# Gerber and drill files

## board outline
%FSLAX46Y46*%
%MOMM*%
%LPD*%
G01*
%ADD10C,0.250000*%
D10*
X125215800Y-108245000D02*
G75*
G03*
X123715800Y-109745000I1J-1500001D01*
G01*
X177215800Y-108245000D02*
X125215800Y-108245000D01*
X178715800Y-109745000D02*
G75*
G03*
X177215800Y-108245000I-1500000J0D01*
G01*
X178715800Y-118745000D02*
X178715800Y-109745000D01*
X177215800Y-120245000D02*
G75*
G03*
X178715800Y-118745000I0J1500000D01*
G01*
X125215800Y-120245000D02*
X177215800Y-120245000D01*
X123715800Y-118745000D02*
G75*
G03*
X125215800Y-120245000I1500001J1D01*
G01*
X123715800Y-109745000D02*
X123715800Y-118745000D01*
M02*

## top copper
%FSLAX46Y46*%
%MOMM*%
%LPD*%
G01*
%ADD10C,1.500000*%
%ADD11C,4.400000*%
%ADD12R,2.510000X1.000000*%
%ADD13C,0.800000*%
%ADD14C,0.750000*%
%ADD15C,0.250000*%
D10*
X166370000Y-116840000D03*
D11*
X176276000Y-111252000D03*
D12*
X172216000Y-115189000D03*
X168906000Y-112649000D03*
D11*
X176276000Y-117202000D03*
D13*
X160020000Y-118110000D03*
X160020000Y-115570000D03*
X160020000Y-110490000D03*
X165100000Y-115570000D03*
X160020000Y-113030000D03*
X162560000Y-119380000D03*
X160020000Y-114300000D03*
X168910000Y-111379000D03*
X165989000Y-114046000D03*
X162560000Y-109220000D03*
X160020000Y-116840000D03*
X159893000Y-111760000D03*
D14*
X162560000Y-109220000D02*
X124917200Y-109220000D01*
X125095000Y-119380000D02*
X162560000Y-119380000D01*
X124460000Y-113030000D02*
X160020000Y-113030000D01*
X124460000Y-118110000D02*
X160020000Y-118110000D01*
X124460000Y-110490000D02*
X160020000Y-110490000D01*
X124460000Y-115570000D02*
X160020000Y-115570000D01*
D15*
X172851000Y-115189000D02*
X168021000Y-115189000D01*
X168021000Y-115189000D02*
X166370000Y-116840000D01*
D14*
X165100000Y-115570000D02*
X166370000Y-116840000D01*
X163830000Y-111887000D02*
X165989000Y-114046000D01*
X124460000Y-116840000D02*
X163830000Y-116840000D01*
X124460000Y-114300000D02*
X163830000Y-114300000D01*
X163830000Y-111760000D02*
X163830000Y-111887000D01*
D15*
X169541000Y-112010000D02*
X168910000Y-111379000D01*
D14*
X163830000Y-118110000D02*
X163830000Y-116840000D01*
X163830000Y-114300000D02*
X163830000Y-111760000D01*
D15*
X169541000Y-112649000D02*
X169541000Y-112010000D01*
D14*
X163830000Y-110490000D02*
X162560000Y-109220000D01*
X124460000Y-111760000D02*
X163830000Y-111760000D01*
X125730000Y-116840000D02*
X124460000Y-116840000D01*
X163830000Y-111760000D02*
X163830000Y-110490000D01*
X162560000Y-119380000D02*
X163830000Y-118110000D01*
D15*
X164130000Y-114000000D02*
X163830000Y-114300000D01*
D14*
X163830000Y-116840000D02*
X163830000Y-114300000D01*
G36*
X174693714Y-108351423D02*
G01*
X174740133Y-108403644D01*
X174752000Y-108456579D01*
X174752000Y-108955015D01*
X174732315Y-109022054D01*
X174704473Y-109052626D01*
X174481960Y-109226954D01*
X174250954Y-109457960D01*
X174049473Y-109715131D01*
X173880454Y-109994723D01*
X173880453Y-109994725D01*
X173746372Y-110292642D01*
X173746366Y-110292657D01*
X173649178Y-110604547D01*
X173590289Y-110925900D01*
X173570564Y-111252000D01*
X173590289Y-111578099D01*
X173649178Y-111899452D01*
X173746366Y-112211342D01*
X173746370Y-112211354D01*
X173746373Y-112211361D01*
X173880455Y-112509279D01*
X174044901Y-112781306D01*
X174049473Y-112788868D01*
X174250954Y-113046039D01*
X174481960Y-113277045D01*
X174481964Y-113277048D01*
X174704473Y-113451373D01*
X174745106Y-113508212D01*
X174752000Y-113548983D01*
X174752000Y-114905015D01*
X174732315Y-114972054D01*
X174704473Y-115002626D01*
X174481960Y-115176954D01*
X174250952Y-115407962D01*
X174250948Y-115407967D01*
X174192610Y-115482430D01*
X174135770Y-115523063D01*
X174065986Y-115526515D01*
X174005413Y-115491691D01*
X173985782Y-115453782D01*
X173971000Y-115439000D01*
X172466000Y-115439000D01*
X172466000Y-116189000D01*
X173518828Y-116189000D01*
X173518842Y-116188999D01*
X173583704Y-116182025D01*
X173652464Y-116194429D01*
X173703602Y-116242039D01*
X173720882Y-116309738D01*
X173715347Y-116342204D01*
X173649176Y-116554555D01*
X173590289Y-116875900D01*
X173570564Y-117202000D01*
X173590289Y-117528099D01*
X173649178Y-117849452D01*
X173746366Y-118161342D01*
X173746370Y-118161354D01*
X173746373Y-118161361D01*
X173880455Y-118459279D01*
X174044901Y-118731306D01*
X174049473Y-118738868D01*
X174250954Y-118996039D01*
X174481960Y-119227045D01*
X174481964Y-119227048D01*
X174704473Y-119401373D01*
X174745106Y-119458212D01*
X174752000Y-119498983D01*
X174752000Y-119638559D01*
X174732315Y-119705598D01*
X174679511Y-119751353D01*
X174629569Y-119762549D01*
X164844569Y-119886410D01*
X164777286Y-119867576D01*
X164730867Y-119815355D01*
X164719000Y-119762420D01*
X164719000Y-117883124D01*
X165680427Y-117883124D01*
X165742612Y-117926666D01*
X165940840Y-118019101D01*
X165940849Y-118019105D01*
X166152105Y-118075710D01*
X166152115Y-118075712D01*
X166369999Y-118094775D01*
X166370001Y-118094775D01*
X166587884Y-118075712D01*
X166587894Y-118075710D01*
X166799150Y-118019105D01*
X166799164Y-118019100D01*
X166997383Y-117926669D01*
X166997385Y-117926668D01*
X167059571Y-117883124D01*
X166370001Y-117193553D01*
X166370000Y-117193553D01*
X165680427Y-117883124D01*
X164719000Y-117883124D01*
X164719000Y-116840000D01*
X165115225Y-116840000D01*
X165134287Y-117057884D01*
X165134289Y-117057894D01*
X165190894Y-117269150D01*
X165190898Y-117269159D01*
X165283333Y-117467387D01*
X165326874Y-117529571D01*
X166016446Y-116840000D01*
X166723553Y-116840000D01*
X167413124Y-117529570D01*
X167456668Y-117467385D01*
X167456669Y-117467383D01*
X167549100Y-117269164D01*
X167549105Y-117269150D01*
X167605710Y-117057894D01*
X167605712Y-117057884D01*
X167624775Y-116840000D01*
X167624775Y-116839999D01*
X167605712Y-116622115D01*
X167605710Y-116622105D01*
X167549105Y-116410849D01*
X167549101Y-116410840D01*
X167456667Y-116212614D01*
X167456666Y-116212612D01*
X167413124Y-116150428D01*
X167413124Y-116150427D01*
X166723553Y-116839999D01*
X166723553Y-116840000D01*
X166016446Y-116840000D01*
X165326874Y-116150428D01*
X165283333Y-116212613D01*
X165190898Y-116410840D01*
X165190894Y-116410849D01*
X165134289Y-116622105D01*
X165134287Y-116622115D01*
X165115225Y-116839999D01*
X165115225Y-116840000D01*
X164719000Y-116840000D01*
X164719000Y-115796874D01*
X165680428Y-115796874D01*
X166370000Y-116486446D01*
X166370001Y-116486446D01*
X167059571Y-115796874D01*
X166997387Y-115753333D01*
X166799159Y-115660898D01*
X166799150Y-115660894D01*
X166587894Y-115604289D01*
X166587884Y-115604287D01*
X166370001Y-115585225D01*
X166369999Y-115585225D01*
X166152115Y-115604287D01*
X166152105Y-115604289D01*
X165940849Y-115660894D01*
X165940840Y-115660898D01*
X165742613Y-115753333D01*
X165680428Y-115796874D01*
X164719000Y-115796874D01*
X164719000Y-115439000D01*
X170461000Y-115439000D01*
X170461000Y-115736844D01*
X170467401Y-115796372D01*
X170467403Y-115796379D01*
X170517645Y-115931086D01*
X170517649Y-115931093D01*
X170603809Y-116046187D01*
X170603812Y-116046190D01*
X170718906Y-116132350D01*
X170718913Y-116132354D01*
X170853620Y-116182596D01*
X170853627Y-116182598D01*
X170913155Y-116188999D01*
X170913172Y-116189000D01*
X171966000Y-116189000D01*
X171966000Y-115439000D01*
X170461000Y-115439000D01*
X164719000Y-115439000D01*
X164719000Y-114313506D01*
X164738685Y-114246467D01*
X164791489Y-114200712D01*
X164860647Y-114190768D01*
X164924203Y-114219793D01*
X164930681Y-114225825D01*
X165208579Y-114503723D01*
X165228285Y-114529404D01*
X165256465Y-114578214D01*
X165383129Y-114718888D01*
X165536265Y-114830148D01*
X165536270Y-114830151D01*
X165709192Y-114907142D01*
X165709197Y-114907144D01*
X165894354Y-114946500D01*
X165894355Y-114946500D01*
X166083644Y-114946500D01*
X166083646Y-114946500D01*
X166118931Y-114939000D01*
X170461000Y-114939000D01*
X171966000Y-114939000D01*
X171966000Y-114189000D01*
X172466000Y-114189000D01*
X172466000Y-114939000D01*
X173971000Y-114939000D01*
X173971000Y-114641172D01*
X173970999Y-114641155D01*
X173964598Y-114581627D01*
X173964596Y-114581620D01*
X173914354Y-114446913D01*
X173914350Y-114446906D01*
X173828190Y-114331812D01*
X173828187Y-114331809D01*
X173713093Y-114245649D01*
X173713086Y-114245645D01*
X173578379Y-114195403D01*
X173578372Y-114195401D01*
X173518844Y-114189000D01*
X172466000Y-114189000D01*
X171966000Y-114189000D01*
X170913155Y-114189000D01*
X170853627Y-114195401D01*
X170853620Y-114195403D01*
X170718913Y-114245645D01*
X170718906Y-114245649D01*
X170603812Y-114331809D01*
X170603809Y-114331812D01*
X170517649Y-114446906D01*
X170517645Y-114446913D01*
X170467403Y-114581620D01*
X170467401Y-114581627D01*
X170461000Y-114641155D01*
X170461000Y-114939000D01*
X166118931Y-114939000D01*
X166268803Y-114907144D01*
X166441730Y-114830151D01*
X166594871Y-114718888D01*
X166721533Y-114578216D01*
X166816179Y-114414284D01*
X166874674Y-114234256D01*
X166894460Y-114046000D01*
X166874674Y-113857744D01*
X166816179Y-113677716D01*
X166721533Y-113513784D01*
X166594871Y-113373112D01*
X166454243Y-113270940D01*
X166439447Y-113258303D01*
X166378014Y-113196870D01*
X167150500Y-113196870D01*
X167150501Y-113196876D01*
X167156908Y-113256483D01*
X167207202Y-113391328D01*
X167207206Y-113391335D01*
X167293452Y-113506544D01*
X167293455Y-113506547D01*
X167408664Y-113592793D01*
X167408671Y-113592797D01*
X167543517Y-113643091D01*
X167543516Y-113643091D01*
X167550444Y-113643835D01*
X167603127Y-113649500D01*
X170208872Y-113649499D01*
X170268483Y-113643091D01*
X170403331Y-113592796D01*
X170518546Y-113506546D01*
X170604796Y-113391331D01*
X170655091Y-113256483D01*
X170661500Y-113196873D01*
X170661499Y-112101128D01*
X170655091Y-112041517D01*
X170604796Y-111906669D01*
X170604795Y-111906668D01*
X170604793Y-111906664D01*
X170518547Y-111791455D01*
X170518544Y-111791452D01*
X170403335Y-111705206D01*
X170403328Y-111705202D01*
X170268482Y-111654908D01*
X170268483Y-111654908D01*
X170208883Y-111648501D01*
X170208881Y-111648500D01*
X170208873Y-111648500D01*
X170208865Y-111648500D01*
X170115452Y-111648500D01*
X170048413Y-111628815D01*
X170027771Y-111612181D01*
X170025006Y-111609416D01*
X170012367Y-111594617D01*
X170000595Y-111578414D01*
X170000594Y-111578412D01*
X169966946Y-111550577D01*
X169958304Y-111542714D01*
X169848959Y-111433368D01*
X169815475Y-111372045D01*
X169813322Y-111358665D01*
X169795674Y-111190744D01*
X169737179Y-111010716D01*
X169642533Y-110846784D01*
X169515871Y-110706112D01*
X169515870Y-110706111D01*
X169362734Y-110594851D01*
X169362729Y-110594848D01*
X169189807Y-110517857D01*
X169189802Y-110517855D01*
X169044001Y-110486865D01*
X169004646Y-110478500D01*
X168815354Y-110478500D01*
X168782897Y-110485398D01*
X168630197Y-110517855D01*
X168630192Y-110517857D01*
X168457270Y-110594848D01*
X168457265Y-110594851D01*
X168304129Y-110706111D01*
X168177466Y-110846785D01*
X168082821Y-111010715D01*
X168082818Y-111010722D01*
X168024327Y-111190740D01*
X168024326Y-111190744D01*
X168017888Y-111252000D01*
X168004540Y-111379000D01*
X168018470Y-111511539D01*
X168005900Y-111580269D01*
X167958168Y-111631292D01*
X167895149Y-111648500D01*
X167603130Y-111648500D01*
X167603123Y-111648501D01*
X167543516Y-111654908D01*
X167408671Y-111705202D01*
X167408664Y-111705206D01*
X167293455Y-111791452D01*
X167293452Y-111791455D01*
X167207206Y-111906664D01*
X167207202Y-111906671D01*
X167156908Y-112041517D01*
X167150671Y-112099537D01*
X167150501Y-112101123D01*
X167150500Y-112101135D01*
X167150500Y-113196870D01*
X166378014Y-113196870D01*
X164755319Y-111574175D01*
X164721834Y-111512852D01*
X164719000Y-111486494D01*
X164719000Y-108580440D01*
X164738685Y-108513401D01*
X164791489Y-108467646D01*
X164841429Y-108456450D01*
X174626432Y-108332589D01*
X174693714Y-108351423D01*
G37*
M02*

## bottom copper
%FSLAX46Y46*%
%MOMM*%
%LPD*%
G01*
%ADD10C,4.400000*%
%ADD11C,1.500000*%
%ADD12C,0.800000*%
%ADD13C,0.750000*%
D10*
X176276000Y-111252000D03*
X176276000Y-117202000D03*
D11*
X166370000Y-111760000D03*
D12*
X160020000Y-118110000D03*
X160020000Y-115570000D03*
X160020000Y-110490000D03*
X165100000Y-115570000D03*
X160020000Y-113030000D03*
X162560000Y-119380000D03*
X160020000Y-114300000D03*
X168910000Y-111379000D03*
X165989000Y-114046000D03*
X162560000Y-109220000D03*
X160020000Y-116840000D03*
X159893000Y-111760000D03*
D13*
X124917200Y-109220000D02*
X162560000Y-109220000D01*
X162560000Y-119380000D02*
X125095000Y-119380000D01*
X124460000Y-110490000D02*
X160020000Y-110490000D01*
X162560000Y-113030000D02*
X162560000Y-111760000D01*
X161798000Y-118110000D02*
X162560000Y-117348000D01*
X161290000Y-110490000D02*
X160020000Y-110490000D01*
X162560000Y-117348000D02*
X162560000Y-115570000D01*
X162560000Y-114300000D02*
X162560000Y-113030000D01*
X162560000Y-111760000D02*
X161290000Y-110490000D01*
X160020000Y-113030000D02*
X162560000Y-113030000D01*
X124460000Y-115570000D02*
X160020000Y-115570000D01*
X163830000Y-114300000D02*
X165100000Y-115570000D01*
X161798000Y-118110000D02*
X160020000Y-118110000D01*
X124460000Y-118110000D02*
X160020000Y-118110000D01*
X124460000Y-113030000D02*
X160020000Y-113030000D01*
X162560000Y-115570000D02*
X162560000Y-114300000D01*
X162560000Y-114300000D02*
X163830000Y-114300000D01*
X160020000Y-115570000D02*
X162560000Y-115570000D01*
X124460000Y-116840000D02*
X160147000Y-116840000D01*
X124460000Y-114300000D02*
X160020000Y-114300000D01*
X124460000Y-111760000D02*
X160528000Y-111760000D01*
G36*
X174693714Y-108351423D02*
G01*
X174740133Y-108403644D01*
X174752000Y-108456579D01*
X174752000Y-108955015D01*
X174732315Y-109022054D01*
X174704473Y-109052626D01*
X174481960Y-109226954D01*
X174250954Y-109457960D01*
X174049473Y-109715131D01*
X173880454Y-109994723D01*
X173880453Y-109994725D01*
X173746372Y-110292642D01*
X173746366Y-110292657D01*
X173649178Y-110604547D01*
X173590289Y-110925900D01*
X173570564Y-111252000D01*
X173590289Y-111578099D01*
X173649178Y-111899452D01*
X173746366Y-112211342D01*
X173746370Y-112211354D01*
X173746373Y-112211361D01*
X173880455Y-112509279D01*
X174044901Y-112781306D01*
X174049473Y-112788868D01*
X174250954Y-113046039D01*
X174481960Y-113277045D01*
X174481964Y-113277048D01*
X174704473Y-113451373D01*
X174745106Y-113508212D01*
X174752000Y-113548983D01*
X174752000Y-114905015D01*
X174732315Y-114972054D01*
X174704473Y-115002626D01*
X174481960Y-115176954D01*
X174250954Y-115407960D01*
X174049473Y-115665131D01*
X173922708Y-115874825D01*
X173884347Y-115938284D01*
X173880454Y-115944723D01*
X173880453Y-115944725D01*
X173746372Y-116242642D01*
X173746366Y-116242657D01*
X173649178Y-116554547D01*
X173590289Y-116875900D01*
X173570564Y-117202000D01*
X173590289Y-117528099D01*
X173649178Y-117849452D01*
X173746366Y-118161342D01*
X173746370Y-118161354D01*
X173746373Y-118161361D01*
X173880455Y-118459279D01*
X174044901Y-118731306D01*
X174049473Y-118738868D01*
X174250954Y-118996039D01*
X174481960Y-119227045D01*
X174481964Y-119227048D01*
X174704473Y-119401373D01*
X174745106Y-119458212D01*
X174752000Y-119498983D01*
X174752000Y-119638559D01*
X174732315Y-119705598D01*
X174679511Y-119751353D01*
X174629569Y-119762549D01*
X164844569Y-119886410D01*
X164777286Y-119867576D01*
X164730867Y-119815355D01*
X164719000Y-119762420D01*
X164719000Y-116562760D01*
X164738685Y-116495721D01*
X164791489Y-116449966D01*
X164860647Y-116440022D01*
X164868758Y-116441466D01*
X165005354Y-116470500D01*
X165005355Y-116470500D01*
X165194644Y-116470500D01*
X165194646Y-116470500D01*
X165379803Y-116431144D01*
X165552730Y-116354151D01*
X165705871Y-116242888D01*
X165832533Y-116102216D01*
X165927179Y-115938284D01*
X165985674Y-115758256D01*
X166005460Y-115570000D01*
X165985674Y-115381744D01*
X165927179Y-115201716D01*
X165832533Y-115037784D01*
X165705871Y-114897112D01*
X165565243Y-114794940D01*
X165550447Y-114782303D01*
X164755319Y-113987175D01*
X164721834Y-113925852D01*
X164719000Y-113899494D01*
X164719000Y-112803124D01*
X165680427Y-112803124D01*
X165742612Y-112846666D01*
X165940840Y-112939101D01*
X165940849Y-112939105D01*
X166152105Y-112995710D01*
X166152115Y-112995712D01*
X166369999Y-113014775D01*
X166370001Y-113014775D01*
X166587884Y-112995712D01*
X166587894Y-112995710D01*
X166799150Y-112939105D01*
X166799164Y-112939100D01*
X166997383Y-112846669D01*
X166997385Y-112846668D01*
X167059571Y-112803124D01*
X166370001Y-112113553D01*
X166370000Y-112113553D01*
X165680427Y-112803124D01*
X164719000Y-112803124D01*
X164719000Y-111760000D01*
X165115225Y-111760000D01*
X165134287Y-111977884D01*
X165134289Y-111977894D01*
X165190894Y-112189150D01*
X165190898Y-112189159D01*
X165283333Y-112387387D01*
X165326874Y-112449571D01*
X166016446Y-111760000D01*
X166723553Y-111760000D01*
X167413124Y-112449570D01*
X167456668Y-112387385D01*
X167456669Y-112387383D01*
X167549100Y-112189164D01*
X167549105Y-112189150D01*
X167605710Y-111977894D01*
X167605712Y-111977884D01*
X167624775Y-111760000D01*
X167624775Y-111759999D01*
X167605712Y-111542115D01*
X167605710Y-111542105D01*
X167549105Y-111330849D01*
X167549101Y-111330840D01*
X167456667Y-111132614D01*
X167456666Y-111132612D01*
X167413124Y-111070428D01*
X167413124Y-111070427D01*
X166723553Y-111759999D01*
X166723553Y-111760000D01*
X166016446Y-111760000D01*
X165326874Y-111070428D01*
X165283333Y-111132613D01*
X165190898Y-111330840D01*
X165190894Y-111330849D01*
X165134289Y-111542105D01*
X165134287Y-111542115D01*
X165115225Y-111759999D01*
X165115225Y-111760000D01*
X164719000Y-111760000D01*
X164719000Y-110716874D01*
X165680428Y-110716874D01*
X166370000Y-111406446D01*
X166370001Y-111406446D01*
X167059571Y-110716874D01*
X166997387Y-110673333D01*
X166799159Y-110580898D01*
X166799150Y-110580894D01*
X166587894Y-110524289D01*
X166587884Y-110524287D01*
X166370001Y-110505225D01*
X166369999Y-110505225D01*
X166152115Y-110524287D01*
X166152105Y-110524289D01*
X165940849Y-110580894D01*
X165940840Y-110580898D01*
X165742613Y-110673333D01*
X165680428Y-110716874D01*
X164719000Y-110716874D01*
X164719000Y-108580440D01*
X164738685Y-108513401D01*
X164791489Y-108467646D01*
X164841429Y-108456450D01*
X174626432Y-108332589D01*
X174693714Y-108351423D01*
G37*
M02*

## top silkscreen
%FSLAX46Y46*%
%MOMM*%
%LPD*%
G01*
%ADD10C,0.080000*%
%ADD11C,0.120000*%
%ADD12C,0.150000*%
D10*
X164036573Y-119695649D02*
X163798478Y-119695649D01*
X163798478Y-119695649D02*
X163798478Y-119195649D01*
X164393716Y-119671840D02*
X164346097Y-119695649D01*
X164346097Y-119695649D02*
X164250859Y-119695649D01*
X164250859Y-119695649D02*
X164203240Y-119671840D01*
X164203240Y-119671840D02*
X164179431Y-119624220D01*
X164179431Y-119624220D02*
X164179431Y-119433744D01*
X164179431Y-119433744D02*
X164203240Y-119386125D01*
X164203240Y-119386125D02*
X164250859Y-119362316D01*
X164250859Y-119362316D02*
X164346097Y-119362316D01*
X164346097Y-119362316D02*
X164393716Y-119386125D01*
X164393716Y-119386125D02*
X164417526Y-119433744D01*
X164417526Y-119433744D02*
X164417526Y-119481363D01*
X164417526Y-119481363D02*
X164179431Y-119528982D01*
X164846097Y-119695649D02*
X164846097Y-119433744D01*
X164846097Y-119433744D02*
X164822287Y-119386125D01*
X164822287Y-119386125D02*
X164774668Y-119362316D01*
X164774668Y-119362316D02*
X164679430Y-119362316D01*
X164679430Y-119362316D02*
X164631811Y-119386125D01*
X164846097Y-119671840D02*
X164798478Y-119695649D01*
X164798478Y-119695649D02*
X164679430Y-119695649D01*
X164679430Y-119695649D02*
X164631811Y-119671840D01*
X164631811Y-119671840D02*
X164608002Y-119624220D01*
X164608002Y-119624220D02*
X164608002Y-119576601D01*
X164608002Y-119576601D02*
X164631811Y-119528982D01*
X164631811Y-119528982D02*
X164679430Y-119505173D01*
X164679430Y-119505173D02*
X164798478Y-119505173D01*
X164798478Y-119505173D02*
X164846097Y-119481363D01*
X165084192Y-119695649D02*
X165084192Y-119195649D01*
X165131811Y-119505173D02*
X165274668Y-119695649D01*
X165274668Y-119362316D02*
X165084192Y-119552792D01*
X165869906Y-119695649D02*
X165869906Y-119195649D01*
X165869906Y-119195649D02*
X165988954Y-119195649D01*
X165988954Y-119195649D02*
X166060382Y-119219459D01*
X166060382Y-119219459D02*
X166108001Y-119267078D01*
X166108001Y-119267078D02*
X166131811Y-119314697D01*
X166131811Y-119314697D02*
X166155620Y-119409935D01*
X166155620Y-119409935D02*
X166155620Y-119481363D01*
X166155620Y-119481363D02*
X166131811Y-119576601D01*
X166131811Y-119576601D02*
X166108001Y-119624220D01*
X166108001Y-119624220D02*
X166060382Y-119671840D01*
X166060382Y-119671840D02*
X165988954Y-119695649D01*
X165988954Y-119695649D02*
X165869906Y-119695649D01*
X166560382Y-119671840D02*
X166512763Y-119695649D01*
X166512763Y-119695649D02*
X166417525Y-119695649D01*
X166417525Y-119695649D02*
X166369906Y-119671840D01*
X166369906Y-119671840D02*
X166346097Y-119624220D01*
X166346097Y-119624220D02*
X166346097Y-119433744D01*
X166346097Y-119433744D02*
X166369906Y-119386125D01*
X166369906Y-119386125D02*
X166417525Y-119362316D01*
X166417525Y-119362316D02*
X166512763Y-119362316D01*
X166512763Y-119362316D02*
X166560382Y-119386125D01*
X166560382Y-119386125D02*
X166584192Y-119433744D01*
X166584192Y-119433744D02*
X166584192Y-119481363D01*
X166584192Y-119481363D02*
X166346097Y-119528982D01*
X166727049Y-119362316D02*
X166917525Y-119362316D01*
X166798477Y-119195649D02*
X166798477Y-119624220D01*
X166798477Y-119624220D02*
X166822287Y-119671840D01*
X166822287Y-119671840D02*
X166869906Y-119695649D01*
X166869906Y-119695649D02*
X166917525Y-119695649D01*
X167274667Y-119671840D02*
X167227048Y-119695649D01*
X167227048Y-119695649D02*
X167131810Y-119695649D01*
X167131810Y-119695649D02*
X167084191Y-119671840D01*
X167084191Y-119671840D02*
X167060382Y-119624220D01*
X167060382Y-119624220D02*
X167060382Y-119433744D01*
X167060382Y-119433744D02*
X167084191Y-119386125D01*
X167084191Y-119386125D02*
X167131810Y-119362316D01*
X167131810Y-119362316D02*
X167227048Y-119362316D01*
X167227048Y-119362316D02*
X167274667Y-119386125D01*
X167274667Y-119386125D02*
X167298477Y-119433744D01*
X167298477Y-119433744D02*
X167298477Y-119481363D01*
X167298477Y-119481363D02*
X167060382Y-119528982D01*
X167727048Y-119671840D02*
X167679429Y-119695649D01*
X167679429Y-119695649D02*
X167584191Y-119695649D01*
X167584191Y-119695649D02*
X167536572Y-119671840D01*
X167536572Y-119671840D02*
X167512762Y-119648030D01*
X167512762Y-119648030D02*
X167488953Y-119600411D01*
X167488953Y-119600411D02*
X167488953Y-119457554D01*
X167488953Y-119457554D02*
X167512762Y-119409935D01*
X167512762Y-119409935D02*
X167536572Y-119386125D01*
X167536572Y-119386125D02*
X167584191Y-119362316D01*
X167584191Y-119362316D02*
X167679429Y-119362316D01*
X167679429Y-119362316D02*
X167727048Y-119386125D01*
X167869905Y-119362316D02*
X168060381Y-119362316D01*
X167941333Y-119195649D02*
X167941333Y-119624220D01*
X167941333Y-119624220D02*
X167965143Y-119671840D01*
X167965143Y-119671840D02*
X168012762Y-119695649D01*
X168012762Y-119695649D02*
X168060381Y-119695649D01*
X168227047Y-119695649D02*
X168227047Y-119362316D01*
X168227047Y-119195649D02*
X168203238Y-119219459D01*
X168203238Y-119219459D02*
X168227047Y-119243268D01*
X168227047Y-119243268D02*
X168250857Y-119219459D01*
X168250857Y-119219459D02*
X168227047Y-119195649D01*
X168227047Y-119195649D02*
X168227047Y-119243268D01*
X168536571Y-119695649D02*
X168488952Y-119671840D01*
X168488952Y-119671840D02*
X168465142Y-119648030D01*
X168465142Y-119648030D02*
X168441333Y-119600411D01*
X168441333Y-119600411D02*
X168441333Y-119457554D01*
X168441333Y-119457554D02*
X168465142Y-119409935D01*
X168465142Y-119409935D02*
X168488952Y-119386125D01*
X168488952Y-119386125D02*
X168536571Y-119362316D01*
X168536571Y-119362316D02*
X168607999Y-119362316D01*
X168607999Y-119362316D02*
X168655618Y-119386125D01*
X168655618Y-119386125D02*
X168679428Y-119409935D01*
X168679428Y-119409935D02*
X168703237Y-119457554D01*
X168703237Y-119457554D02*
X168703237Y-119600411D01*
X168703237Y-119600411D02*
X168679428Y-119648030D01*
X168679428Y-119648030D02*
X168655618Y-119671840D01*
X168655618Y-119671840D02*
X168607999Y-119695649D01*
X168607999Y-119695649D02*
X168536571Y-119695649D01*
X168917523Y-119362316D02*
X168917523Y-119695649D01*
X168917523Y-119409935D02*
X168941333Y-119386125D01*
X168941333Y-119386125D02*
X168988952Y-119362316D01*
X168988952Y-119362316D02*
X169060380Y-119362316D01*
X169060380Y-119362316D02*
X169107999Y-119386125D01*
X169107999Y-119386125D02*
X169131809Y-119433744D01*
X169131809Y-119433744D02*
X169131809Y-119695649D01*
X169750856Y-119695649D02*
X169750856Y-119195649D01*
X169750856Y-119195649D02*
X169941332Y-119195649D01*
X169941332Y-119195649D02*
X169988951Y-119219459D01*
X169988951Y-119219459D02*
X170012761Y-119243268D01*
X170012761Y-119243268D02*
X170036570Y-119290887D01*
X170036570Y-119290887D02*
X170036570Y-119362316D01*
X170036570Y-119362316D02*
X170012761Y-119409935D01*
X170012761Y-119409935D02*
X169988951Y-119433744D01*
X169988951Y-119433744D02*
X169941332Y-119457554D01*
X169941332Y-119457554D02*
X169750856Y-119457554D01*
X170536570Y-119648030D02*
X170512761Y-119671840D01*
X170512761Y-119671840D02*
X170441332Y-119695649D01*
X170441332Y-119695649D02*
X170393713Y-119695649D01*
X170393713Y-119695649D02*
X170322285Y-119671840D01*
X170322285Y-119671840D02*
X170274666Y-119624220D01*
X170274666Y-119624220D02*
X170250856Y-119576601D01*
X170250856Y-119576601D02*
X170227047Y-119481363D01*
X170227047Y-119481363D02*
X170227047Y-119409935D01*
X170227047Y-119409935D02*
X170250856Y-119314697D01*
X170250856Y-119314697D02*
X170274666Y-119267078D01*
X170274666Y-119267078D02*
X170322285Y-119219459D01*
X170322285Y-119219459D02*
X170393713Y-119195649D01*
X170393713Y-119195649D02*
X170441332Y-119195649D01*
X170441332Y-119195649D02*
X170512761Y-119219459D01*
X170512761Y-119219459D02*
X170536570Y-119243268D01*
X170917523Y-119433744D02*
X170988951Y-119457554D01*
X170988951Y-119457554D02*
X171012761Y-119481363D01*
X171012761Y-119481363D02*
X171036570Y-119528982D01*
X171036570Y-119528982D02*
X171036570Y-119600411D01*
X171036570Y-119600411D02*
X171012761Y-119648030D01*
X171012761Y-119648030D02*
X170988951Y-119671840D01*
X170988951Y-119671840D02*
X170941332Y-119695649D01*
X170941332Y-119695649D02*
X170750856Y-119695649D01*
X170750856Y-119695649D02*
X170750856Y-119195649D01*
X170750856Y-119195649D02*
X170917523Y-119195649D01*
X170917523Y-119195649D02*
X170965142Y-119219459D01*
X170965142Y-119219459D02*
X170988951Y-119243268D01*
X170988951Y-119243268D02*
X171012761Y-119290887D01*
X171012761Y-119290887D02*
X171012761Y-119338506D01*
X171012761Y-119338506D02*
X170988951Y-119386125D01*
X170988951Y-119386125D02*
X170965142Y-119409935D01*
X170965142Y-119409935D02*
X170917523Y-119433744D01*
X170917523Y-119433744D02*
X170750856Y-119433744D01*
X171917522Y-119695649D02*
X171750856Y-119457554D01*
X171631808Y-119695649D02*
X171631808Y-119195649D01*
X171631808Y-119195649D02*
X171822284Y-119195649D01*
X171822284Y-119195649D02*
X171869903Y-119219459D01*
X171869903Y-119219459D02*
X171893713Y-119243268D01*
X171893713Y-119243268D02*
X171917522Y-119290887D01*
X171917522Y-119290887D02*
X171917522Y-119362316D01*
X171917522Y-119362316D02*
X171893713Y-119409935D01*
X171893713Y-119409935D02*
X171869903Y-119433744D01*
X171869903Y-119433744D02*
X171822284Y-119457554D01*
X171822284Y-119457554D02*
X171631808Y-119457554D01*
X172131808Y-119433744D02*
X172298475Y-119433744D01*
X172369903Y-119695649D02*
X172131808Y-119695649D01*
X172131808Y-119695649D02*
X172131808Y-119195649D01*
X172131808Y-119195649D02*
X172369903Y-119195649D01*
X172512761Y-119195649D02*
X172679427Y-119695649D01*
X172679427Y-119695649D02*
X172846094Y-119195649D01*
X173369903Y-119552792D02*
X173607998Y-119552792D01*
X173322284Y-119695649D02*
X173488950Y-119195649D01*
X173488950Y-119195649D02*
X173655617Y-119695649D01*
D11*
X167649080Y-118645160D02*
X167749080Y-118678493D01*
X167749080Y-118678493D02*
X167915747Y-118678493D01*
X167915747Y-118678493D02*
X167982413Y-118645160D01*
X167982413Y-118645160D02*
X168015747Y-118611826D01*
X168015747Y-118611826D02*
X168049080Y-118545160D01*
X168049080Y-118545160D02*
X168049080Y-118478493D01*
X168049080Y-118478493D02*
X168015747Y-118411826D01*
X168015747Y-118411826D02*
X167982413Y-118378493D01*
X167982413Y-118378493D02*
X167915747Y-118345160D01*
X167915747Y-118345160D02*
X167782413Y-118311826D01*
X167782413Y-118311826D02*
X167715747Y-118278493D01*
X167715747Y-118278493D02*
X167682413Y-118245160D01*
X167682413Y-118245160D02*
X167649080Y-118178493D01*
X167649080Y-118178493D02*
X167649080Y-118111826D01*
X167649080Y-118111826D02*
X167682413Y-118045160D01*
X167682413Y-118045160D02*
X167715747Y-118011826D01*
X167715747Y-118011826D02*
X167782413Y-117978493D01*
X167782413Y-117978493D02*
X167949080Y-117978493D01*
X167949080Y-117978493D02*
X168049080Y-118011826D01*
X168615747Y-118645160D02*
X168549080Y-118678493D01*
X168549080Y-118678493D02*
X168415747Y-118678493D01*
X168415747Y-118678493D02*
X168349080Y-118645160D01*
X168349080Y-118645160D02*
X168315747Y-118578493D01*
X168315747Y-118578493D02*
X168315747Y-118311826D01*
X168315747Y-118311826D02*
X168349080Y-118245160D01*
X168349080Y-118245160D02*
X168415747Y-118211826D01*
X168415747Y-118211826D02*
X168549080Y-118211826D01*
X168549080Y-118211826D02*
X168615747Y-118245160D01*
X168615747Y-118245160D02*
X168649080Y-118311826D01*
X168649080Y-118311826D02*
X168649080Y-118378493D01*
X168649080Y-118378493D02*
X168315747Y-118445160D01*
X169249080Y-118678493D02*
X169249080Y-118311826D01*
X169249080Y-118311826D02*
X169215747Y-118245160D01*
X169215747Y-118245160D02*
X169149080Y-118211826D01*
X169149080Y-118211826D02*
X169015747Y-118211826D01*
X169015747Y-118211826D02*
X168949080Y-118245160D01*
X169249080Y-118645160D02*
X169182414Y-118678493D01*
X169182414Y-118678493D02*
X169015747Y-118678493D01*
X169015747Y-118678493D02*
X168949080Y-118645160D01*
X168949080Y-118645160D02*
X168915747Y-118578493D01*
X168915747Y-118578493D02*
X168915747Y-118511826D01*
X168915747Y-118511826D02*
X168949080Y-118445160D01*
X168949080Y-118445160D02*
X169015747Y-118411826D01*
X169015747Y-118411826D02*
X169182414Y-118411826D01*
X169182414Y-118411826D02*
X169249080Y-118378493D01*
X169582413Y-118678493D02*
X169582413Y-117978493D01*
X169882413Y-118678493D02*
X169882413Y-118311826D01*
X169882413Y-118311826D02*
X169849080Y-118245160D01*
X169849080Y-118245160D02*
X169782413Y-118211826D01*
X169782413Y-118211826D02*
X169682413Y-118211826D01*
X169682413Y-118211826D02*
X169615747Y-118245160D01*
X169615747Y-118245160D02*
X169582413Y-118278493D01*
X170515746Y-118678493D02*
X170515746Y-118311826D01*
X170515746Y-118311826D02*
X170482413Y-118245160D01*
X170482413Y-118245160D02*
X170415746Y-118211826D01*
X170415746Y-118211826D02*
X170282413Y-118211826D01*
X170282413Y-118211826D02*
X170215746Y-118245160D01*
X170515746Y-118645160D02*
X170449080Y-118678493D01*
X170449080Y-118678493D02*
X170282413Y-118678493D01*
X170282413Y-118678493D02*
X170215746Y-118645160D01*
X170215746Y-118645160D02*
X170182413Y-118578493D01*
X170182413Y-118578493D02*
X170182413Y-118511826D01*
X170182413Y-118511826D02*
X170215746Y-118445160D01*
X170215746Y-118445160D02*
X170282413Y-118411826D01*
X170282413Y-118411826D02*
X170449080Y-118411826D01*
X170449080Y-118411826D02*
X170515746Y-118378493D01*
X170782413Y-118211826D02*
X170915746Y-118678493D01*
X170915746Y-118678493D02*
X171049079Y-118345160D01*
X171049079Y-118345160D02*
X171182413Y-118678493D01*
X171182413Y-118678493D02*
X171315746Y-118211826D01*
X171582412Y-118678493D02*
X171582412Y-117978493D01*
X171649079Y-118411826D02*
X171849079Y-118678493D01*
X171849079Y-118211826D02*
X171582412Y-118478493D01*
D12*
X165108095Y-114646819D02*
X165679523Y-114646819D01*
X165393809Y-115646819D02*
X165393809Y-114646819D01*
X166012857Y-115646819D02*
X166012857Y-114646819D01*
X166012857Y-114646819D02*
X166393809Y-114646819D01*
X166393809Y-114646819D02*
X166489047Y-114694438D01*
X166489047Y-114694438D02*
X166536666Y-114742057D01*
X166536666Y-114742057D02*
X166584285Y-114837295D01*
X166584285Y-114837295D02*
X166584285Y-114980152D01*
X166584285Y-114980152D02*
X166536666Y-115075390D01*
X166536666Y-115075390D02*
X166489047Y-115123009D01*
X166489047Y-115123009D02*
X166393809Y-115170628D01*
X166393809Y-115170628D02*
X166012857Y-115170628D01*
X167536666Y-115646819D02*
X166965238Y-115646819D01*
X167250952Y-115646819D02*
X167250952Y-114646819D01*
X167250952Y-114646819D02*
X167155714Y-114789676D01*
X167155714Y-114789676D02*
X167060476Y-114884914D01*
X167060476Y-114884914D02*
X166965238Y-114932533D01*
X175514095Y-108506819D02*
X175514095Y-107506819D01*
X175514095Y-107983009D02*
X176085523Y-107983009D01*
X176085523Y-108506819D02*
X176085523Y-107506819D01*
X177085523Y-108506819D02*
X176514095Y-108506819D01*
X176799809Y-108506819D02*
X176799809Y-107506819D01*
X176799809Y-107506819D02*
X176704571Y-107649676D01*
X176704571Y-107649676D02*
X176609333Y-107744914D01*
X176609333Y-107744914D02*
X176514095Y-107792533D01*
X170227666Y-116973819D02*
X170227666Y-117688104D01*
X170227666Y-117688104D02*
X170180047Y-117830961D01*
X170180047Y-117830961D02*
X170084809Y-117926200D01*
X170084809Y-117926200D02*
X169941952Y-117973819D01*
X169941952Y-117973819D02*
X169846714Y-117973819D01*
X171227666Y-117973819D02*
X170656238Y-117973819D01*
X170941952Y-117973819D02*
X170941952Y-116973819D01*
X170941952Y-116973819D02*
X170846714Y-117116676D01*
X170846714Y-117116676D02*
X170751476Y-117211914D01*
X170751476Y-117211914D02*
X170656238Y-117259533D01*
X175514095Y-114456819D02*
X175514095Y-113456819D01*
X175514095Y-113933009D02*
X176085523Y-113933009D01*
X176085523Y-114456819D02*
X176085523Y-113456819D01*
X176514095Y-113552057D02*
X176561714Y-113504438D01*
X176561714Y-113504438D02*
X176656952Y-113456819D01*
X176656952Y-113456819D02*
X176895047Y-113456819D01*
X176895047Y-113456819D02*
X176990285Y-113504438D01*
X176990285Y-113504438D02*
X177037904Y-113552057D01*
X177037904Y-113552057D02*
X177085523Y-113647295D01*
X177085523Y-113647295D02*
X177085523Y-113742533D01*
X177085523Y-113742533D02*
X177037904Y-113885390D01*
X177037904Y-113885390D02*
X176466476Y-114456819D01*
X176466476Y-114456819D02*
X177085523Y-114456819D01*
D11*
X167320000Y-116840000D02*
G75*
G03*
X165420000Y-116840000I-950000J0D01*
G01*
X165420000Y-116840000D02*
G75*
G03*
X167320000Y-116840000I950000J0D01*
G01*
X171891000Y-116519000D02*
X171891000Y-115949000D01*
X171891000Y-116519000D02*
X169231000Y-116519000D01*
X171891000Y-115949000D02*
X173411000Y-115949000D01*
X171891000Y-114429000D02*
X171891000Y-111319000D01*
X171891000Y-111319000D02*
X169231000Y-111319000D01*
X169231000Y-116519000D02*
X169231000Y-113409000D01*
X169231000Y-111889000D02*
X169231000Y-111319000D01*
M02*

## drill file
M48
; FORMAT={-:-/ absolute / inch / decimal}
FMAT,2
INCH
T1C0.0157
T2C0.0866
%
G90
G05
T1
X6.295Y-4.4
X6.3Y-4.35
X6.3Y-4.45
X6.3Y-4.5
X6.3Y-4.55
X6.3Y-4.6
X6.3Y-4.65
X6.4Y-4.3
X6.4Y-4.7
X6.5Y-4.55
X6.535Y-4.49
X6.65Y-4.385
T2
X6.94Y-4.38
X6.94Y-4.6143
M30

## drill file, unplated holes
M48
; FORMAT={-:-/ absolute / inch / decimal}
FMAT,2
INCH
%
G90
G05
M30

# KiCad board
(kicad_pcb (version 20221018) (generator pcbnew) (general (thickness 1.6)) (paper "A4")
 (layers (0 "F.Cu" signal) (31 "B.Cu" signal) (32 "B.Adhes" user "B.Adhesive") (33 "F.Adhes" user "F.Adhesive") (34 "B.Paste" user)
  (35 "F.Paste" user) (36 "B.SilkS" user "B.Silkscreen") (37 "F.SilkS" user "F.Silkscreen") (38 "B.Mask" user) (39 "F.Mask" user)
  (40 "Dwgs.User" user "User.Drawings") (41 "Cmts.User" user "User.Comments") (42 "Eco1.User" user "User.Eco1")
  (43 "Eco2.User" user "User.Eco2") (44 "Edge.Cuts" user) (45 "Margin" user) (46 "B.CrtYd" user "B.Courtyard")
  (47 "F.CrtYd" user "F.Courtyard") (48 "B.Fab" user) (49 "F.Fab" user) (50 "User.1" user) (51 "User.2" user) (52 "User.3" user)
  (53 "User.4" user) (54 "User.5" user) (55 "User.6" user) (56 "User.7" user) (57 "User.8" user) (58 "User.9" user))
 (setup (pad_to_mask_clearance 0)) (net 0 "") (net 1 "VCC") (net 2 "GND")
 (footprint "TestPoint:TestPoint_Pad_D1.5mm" (layer "F.Cu") (at 166.37 116.84)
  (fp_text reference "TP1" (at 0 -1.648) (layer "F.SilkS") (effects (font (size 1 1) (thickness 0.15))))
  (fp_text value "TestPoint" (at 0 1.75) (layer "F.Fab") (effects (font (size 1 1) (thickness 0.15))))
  (fp_circle (center 0 0) (end 0 0.95) (stroke (width 0.12) (type solid)) (fill none) (layer "F.SilkS"))
  (pad "1" smd circle (at 0 0) (size 1.5 1.5) (layers "F.Cu" "F.Mask") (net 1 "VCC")))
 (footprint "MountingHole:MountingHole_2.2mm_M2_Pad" (layer "F.Cu") (at 176.276 111.252)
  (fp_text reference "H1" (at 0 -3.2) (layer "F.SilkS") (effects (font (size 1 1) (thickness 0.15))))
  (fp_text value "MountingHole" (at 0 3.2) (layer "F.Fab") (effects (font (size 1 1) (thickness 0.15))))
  (pad "1" thru_hole circle (at 0 0) (size 4.4 4.4) (drill 2.2) (layers "*.Cu" "*.Mask")))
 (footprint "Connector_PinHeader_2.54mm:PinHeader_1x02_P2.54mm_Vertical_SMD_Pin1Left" (layer "F.Cu") (at 170.561 113.919 180)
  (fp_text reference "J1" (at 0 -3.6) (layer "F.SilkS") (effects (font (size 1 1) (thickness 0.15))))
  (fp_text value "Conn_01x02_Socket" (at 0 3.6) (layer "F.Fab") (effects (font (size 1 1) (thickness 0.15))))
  (fp_line (start -1.33 -2.6) (end -1.33 -2.03) (stroke (width 0.12) (type solid)) (layer "F.SilkS"))
  (fp_line (start -1.33 -2.6) (end 1.33 -2.6) (stroke (width 0.12) (type solid)) (layer "F.SilkS"))
  (fp_line (start -1.33 -2.03) (end -2.85 -2.03) (stroke (width 0.12) (type solid)) (layer "F.SilkS"))
  (fp_line (start -1.33 -0.51) (end -1.33 2.6) (stroke (width 0.12) (type solid)) (layer "F.SilkS"))
  (fp_line (start -1.33 2.6) (end 1.33 2.6) (stroke (width 0.12) (type solid)) (layer "F.SilkS"))
  (fp_line (start 1.33 -2.6) (end 1.33 0.51) (stroke (width 0.12) (type solid)) (layer "F.SilkS"))
  (fp_line (start 1.33 2.03) (end 1.33 2.6) (stroke (width 0.12) (type solid)) (layer "F.SilkS"))
  (pad "1" smd rect (at -1.655 -1.27 180) (size 2.51 1) (layers "F.Cu" "F.Paste" "F.Mask") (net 1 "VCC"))
  (pad "2" smd rect (at 1.655 1.27 180) (size 2.51 1) (layers "F.Cu" "F.Paste" "F.Mask") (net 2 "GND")))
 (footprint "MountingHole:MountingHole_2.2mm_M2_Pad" (layer "F.Cu") (at 176.276 117.202)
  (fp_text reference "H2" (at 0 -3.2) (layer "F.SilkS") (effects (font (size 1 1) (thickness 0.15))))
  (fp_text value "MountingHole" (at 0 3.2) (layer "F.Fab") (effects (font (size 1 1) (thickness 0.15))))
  (pad "1" thru_hole circle (at 0 0) (size 4.4 4.4) (drill 2.2) (layers "*.Cu" "*.Mask")))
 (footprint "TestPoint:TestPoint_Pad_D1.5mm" (layer "B.Cu") (at 166.37 111.76 180)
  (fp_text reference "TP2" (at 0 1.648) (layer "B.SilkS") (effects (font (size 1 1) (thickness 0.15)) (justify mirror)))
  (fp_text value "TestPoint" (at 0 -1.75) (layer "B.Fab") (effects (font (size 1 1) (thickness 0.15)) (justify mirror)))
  (pad "1" smd circle (at 0 0 180) (size 1.5 1.5) (layers "B.Cu" "B.Mask") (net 2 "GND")))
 (gr_arc (start 123.7158 109.745) (mid 124.15514 108.68434) (end 125.2158 108.245) (stroke (width 0.25) (type solid)) (layer "Edge.Cuts"))
 (gr_arc (start 125.2158 120.245) (mid 124.15514 119.80566) (end 123.7158 118.745) (stroke (width 0.25) (type solid)) (layer "Edge.Cuts"))
 (gr_line (start 125.2158 120.245) (end 177.2158 120.245) (stroke (width 0.25) (type solid)) (layer "Edge.Cuts"))
 (gr_line (start 123.7158 109.745) (end 123.7158 118.745) (stroke (width 0.25) (type solid)) (layer "Edge.Cuts"))
 (gr_arc (start 178.7158 118.745) (mid 178.27646 119.80566) (end 177.2158 120.245) (stroke (width 0.25) (type solid)) (layer "Edge.Cuts"))
 (gr_line (start 178.7158 118.745) (end 178.7158 109.745) (stroke (width 0.25) (type solid)) (layer "Edge.Cuts"))
 (gr_arc (start 177.2158 108.245) (mid 178.27646 108.68434) (end 178.7158 109.745) (stroke (width 0.25) (type solid)) (layer "Edge.Cuts"))
 (gr_line (start 177.2158 108.245) (end 125.2158 108.245) (stroke (width 0.25) (type solid)) (layer "Edge.Cuts"))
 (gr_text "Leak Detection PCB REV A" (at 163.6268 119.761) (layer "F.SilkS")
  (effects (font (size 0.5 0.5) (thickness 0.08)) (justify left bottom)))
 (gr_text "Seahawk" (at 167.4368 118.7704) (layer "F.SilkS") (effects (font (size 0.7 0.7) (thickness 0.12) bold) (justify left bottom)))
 (segment (start 124.46 113.03) (end 160.02 113.03) (width 0.75) (layer "F.Cu") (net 1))
 (segment (start 124.46 118.11) (end 160.02 118.11) (width 0.75) (layer "F.Cu") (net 1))
 (segment (start 124.46 110.49) (end 160.02 110.49) (width 0.75) (layer "F.Cu") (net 1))
 (segment (start 124.46 115.57) (end 160.02 115.57) (width 0.75) (layer "F.Cu") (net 1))
 (segment (start 172.851 115.189) (end 168.021 115.189) (width 0.25) (layer "F.Cu") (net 1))
 (segment (start 168.021 115.189) (end 166.37 116.84) (width 0.25) (layer "F.Cu") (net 1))
 (segment (start 165.1 115.57) (end 166.37 116.84) (width 0.75) (layer "F.Cu") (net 1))
 (via (at 160.02 118.11) (size 0.8) (drill 0.4) (layers "F.Cu" "B.Cu") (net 1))
 (via (at 160.02 115.57) (size 0.8) (drill 0.4) (layers "F.Cu" "B.Cu") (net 1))
 (via (at 160.02 110.49) (size 0.8) (drill 0.4) (layers "F.Cu" "B.Cu") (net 1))
 (via (at 165.1 115.57) (size 0.8) (drill 0.4) (layers "F.Cu" "B.Cu") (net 1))
 (via (at 160.02 113.03) (size 0.8) (drill 0.4) (layers "F.Cu" "B.Cu") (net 1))
 (segment (start 124.46 110.49) (end 160.02 110.49) (width 0.75) (layer "B.Cu") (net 1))
 (segment (start 162.56 113.03) (end 162.56 111.76) (width 0.75) (layer "B.Cu") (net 1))
 (segment (start 161.798 118.11) (end 162.56 117.348) (width 0.75) (layer "B.Cu") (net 1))
 (segment (start 161.29 110.49) (end 160.02 110.49) (width 0.75) (layer "B.Cu") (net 1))
 (segment (start 162.56 117.348) (end 162.56 115.57) (width 0.75) (layer "B.Cu") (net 1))
 (segment (start 162.56 114.3) (end 162.56 113.03) (width 0.75) (layer "B.Cu") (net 1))
 (segment (start 162.56 111.76) (end 161.29 110.49) (width 0.75) (layer "B.Cu") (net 1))
 (segment (start 160.02 113.03) (end 162.56 113.03) (width 0.75) (layer "B.Cu") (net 1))
 (segment (start 124.46 115.57) (end 160.02 115.57) (width 0.75) (layer "B.Cu") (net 1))
 (segment (start 163.83 114.3) (end 165.1 115.57) (width 0.75) (layer "B.Cu") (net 1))
 (segment (start 161.798 118.11) (end 160.02 118.11) (width 0.75) (layer "B.Cu") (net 1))
 (segment (start 124.46 118.11) (end 160.02 118.11) (width 0.75) (layer "B.Cu") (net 1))
 (segment (start 124.46 113.03) (end 160.02 113.03) (width 0.75) (layer "B.Cu") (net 1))
 (segment (start 162.56 115.57) (end 162.56 114.3) (width 0.75) (layer "B.Cu") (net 1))
 (segment (start 162.56 114.3) (end 163.83 114.3) (width 0.75) (layer "B.Cu") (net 1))
 (segment (start 160.02 115.57) (end 162.56 115.57) (width 0.75) (layer "B.Cu") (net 1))
 (segment (start 163.83 111.887) (end 165.989 114.046) (width 0.75) (layer "F.Cu") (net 2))
 (segment (start 124.46 116.84) (end 163.83 116.84) (width 0.75) (layer "F.Cu") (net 2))
 (segment (start 124.46 114.3) (end 163.83 114.3) (width 0.75) (layer "F.Cu") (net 2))
 (segment (start 163.83 111.76) (end 163.83 111.887) (width 0.75) (layer "F.Cu") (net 2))
 (segment (start 169.541 112.01) (end 168.91 111.379) (width 0.25) (layer "F.Cu") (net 2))
 (segment (start 163.83 118.11) (end 163.83 116.84) (width 0.75) (layer "F.Cu") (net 2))
 (segment (start 163.83 114.3) (end 163.83 111.76) (width 0.75) (layer "F.Cu") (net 2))
 (segment (start 162.56 109.22) (end 124.9172 109.22) (width 0.75) (layer "F.Cu") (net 2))
 (segment (start 169.541 112.649) (end 169.541 112.01) (width 0.25) (layer "F.Cu") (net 2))
 (segment (start 125.095 119.38) (end 162.56 119.38) (width 0.75) (layer "F.Cu") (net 2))
 (segment (start 163.83 110.49) (end 162.56 109.22) (width 0.75) (layer "F.Cu") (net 2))
 (segment (start 124.46 111.76) (end 163.83 111.76) (width 0.75) (layer "F.Cu") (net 2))
 (segment (start 125.73 116.84) (end 124.46 116.84) (width 0.75) (layer "F.Cu") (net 2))
 (segment (start 163.83 111.76) (end 163.83 110.49) (width 0.75) (layer "F.Cu") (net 2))
 (segment (start 162.56 119.38) (end 163.83 118.11) (width 0.75) (layer "F.Cu") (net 2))
 (segment (start 164.13 114) (end 163.83 114.3) (width 0.25) (layer "F.Cu") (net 2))
 (segment (start 163.83 116.84) (end 163.83 114.3) (width 0.75) (layer "F.Cu") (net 2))
 (via (at 162.56 119.38) (size 0.8) (drill 0.4) (layers "F.Cu" "B.Cu") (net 2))
 (via (at 160.02 114.3) (size 0.8) (drill 0.4) (layers "F.Cu" "B.Cu") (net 2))
 (via (at 168.91 111.379) (size 0.8) (drill 0.4) (layers "F.Cu" "B.Cu") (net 2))
 (via (at 165.989 114.046) (size 0.8) (drill 0.4) (layers "F.Cu" "B.Cu") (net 2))
 (via (at 162.56 109.22) (size 0.8) (drill 0.4) (layers "F.Cu" "B.Cu") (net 2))
 (via (at 160.02 116.84) (size 0.8) (drill 0.4) (layers "F.Cu" "B.Cu") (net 2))
 (via (at 159.893 111.76) (size 0.8) (drill 0.4) (layers "F.Cu" "B.Cu") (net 2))
 (segment (start 124.46 116.84) (end 160.147 116.84) (width 0.75) (layer "B.Cu") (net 2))
 (segment (start 124.9172 109.22) (end 162.56 109.22) (width 0.75) (layer "B.Cu") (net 2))
 (segment (start 162.56 119.38) (end 125.095 119.38) (width 0.75) (layer "B.Cu") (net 2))
 (segment (start 124.46 114.3) (end 160.02 114.3) (width 0.75) (layer "B.Cu") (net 2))
 (segment (start 124.46 111.76) (end 160.528 111.76) (width 0.75) (layer "B.Cu") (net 2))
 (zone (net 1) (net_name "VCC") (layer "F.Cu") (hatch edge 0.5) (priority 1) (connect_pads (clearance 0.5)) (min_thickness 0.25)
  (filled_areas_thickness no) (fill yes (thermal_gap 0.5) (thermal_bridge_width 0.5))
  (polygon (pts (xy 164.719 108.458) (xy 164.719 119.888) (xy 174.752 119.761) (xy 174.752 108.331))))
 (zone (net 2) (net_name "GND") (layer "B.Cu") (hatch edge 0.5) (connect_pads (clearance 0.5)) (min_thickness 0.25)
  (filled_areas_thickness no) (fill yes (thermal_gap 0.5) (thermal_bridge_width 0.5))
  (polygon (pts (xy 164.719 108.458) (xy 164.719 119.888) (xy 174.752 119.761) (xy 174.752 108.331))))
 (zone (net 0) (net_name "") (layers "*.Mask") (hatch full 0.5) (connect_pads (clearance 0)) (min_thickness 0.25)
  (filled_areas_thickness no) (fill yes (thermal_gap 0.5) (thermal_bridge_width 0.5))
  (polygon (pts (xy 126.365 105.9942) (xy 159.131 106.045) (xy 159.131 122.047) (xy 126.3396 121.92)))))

